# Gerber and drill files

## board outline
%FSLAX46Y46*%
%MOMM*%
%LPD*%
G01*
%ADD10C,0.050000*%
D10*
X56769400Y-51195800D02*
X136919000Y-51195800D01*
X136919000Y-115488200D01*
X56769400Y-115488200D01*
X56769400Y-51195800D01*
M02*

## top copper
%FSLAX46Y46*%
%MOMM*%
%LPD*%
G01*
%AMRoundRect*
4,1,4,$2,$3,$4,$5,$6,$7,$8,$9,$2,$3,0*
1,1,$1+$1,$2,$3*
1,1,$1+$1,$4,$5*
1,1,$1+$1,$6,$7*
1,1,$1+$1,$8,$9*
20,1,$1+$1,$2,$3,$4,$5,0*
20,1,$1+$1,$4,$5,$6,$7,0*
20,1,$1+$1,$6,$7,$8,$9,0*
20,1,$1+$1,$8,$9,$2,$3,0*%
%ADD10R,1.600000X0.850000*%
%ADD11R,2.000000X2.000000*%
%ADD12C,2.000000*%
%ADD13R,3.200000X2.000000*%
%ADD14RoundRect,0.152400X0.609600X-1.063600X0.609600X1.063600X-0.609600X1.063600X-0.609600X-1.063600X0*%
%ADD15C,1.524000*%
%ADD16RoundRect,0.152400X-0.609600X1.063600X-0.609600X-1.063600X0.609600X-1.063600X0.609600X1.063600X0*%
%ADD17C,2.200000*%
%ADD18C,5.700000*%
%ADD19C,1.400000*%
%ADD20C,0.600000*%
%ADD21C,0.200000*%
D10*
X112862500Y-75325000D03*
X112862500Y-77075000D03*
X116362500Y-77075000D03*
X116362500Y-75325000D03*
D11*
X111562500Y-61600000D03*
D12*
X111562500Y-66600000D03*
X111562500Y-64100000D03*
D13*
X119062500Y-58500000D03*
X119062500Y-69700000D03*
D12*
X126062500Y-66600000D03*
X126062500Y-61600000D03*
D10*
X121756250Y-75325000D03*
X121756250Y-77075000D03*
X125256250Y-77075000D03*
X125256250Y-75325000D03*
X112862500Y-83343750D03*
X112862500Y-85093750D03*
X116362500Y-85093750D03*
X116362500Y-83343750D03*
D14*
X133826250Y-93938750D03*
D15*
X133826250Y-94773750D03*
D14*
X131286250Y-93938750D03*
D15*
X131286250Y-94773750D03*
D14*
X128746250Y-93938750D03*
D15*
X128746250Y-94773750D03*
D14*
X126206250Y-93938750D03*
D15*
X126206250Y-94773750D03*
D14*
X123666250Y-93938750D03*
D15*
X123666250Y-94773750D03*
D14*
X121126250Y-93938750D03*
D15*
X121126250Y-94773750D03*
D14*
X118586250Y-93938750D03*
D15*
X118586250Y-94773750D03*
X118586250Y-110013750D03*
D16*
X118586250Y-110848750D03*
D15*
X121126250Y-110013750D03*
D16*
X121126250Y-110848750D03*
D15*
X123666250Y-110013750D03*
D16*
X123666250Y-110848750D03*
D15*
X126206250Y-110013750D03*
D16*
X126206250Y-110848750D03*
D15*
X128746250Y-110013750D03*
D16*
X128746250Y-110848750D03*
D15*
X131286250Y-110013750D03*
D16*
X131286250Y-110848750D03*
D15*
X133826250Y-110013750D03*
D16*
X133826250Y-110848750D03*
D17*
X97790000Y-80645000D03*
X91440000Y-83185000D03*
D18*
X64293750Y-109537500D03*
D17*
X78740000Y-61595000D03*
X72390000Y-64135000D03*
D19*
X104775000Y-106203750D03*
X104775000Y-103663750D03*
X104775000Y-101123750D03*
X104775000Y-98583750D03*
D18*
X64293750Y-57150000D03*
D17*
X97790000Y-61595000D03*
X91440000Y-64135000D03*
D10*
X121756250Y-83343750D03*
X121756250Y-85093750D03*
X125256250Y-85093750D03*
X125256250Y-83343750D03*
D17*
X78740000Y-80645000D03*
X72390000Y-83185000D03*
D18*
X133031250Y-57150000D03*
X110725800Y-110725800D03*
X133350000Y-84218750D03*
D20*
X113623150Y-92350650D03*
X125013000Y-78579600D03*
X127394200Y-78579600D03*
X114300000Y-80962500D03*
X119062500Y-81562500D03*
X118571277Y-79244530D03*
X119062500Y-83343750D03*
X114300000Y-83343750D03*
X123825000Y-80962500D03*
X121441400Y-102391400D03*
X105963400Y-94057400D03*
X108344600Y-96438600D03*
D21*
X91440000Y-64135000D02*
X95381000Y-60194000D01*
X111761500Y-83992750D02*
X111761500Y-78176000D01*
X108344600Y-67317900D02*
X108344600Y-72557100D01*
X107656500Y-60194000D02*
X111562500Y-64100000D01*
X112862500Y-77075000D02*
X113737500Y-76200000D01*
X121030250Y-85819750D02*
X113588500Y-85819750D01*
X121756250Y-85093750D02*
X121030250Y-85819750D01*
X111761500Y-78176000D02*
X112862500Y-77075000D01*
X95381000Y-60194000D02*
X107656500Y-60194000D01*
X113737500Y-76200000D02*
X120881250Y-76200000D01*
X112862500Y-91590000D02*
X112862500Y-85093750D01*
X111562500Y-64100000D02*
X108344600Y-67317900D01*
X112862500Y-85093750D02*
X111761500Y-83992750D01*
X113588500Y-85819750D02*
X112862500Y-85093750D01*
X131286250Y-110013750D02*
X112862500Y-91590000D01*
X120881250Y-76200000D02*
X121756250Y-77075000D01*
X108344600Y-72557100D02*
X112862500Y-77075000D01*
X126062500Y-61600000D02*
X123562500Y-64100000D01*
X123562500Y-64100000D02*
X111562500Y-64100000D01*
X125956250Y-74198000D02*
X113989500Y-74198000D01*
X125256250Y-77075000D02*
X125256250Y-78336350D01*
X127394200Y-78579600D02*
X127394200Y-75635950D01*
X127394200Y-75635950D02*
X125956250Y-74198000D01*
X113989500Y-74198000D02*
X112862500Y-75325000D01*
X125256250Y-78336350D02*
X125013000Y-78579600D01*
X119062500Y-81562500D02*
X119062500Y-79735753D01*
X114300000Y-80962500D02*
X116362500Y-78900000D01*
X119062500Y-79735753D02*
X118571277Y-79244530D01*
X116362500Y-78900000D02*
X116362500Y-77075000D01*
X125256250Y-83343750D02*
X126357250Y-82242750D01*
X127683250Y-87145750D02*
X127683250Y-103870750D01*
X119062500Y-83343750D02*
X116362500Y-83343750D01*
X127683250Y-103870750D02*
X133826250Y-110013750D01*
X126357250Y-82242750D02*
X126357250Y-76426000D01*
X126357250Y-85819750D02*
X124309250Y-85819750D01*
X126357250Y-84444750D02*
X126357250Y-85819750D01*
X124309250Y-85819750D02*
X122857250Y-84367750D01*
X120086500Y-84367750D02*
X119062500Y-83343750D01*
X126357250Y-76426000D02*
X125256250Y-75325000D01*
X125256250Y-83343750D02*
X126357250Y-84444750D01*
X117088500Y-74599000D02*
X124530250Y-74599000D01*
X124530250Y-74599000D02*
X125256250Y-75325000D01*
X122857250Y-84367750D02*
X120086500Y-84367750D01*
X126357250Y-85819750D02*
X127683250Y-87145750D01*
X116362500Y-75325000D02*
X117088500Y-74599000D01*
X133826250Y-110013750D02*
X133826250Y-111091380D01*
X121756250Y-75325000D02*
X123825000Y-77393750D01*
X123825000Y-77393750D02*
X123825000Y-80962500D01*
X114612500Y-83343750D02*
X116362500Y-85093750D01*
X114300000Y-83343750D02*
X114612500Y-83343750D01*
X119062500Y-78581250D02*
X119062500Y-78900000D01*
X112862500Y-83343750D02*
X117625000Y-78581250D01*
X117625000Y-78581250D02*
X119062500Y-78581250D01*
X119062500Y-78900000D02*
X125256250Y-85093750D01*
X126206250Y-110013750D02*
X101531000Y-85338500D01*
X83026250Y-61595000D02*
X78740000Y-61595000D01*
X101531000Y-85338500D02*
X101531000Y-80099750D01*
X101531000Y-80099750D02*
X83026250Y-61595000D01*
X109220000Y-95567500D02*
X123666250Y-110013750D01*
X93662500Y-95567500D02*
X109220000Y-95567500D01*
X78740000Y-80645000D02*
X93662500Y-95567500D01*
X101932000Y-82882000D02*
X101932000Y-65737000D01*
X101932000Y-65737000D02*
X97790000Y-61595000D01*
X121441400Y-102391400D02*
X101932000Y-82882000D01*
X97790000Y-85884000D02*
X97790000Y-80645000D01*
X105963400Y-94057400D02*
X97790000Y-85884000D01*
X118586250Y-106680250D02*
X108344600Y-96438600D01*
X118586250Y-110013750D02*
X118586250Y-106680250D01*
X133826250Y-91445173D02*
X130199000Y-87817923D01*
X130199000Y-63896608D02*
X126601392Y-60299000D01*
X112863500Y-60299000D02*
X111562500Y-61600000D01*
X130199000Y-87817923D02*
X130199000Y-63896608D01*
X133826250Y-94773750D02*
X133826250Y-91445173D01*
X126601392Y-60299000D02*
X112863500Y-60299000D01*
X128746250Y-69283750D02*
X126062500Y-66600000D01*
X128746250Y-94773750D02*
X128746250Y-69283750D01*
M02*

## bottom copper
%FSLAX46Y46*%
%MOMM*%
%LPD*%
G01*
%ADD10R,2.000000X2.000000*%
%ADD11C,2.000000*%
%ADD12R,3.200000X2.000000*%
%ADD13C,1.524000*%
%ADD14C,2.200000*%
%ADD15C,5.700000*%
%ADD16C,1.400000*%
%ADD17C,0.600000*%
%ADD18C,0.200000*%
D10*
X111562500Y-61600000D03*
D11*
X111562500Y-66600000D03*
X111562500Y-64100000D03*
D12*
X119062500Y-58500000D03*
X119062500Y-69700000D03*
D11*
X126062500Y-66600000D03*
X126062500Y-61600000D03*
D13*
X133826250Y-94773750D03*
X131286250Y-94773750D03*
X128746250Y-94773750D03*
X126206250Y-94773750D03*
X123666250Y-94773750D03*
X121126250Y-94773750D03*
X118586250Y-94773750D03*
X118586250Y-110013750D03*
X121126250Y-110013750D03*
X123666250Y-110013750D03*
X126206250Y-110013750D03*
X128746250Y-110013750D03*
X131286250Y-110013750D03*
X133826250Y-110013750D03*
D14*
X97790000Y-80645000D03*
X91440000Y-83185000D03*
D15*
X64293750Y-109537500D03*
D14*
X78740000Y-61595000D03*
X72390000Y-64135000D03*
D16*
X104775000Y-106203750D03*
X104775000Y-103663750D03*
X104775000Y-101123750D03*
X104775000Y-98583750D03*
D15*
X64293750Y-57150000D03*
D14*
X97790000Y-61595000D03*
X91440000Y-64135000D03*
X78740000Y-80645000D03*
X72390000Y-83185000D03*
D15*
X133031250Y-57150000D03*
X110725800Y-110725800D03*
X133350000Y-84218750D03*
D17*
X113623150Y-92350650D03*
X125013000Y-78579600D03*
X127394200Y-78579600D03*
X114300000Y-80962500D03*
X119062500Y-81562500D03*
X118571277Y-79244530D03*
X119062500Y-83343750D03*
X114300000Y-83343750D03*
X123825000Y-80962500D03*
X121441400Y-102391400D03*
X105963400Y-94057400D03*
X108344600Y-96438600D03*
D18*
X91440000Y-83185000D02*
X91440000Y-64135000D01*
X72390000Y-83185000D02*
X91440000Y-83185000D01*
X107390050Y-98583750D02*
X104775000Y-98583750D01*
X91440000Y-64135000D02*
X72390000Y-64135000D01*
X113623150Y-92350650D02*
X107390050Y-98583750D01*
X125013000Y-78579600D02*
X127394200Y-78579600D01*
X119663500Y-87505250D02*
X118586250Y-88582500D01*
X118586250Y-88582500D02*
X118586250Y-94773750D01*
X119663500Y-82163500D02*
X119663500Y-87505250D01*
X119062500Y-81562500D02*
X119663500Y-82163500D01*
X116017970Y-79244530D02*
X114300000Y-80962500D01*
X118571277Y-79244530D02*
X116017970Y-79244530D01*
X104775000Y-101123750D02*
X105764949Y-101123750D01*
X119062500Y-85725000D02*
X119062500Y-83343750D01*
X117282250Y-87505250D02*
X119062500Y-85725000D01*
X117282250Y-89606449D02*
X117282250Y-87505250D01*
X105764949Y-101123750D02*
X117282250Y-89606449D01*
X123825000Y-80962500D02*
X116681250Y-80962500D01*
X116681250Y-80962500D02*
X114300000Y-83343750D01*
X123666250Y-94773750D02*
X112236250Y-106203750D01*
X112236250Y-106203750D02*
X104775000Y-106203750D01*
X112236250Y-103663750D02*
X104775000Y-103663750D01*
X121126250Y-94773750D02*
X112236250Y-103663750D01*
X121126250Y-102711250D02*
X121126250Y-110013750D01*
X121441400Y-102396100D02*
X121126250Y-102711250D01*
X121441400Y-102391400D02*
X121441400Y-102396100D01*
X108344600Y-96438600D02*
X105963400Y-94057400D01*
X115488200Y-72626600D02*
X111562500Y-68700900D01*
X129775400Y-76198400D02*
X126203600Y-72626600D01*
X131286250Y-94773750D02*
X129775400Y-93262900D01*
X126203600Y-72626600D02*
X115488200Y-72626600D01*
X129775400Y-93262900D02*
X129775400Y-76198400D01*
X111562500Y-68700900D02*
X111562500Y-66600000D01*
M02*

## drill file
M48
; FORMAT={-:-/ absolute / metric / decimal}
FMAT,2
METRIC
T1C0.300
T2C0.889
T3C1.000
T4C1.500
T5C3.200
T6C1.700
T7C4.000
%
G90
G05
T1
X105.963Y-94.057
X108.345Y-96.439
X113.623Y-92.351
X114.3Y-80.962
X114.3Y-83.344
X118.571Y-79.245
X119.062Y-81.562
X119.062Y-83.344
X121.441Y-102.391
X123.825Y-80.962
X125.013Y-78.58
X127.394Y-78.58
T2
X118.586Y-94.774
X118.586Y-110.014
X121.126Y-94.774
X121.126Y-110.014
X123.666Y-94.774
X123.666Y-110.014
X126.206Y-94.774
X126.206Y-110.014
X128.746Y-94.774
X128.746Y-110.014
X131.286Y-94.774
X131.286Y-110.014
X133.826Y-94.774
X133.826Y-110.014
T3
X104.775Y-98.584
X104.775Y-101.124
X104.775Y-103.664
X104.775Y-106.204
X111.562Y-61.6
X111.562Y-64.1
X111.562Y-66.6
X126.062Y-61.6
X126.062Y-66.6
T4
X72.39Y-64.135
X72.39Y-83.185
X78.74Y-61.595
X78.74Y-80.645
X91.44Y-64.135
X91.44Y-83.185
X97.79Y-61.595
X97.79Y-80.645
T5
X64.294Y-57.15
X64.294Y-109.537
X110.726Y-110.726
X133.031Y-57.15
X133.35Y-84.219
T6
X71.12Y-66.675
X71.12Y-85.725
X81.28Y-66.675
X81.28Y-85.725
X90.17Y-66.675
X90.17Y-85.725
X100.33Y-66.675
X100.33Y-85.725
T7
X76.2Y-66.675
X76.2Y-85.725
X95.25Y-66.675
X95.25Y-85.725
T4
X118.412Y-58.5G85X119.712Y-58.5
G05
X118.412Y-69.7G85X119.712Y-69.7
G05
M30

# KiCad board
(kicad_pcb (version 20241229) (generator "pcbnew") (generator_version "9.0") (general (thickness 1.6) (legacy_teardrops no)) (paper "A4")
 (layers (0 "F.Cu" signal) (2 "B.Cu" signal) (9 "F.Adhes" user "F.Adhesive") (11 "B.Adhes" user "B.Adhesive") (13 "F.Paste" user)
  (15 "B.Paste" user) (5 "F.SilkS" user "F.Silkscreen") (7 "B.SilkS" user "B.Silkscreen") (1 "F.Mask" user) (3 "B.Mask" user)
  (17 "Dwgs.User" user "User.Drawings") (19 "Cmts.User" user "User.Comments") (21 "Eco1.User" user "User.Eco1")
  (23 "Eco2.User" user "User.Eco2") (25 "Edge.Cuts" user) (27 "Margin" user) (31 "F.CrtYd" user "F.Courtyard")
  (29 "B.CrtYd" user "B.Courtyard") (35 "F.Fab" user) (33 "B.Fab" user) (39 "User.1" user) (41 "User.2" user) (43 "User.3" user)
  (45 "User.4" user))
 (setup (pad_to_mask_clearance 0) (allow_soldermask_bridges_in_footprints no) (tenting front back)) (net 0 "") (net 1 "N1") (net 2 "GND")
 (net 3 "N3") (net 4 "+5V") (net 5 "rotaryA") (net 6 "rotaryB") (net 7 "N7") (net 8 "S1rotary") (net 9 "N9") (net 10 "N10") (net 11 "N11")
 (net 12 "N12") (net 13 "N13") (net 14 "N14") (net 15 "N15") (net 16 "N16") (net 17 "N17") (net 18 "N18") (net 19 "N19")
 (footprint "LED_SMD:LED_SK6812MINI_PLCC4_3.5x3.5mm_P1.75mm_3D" (layer "F.Cu") (at 114.6125 76.2)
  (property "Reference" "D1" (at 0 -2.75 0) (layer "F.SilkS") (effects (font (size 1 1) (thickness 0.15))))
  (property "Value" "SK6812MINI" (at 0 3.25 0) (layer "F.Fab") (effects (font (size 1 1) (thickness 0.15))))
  (pad "1" smd rect (at -1.75 -0.875) (size 1.6 0.85) (layers "F.Cu" "F.Mask" "F.Paste") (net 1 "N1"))
  (pad "2" smd rect (at -1.75 0.875) (size 1.6 0.85) (layers "F.Cu" "F.Mask" "F.Paste") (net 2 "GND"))
  (pad "3" smd rect (at 1.75 0.875) (size 1.6 0.85) (layers "F.Cu" "F.Mask" "F.Paste") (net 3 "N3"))
  (pad "4" smd rect (at 1.75 -0.875) (size 1.6 0.85) (layers "F.Cu" "F.Mask" "F.Paste") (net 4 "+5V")))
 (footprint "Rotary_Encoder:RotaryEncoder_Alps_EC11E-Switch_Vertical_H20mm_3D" (layer "F.Cu") (at 111.5625 61.6)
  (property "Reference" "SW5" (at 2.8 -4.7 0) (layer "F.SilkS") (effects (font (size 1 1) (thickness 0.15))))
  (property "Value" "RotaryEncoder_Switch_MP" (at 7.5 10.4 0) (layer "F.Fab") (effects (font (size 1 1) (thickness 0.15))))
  (pad "A" thru_hole rect (at 0 0) (size 2 2) (drill 1) (layers "*.Cu" "*.Mask") (remove_unused_layers no) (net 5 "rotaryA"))
  (pad "B" thru_hole circle (at 0 5) (size 2 2) (drill 1) (layers "*.Cu" "*.Mask") (remove_unused_layers no) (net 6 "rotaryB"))
  (pad "C" thru_hole circle (at 0 2.5) (size 2 2) (drill 1) (layers "*.Cu" "*.Mask") (remove_unused_layers no) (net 2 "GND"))
  (pad "MP" thru_hole rect (at 7.5 -3.1) (size 3.2 2) (drill oval 2.8 1.5) (layers "*.Cu" "*.Mask") (remove_unused_layers no) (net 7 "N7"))
  (pad "MP" thru_hole rect (at 7.5 8.1) (size 3.2 2) (drill oval 2.8 1.5) (layers "*.Cu" "*.Mask") (remove_unused_layers no) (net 7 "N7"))
  (pad "S1" thru_hole circle (at 14.5 5) (size 2 2) (drill 1) (layers "*.Cu" "*.Mask") (remove_unused_layers no) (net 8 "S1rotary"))
  (pad "S2" thru_hole circle (at 14.5 0) (size 2 2) (drill 1) (layers "*.Cu" "*.Mask") (remove_unused_layers no) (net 2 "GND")))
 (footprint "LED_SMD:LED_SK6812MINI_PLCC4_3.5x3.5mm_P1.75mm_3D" (layer "F.Cu") (at 123.50625 76.2)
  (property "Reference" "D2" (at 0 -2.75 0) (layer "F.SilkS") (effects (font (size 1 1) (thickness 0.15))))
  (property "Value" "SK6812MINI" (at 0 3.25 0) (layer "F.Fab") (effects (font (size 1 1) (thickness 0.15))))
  (pad "1" smd rect (at -1.75 -0.875) (size 1.6 0.85) (layers "F.Cu" "F.Mask" "F.Paste") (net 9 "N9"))
  (pad "2" smd rect (at -1.75 0.875) (size 1.6 0.85) (layers "F.Cu" "F.Mask" "F.Paste") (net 2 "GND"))
  (pad "3" smd rect (at 1.75 0.875) (size 1.6 0.85) (layers "F.Cu" "F.Mask" "F.Paste") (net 1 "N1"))
  (pad "4" smd rect (at 1.75 -0.875) (size 1.6 0.85) (layers "F.Cu" "F.Mask" "F.Paste") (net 4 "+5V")))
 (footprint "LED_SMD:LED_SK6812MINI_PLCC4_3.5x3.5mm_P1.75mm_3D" (layer "F.Cu") (at 114.6125 84.21875)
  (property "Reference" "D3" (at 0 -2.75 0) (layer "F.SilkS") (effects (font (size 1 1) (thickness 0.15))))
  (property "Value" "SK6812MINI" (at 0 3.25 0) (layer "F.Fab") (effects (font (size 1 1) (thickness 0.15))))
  (pad "1" smd rect (at -1.75 -0.875) (size 1.6 0.85) (layers "F.Cu" "F.Mask" "F.Paste") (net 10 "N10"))
  (pad "2" smd rect (at -1.75 0.875) (size 1.6 0.85) (layers "F.Cu" "F.Mask" "F.Paste") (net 2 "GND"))
  (pad "3" smd rect (at 1.75 0.875) (size 1.6 0.85) (layers "F.Cu" "F.Mask" "F.Paste") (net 9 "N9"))
  (pad "4" smd rect (at 1.75 -0.875) (size 1.6 0.85) (layers "F.Cu" "F.Mask" "F.Paste") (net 4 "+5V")))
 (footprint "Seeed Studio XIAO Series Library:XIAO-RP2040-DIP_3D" (layer "F.Cu") (at 126.20625 102.39375 -90)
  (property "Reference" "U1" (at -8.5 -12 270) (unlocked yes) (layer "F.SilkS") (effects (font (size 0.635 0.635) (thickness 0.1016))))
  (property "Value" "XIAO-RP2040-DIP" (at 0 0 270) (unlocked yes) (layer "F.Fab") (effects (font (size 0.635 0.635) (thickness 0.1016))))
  (pad "1" smd roundrect (at -8.455 -7.62 90) (size 2.432 1.524) (layers "F.Cu" "F.Mask") (roundrect_rratio 0.1) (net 5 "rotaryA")
   (thermal_bridge_angle 45))
  (pad "1" thru_hole circle (at -7.62 -7.62 90) (size 1.524 1.524) (drill 0.889) (layers "*.Cu" "*.Mask") (remove_unused_layers no)
   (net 5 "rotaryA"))
  (pad "2" smd roundrect (at -8.455 -5.08 90) (size 2.432 1.524) (layers "F.Cu" "F.Mask") (roundrect_rratio 0.1) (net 6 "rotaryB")
   (thermal_bridge_angle 45))
  (pad "2" thru_hole circle (at -7.62 -5.08 90) (size 1.524 1.524) (drill 0.889) (layers "*.Cu" "*.Mask") (remove_unused_layers no)
   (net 6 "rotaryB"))
  (pad "3" smd roundrect (at -8.455 -2.54 90) (size 2.432 1.524) (layers "F.Cu" "F.Mask") (roundrect_rratio 0.1) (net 8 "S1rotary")
   (thermal_bridge_angle 45))
  (pad "3" thru_hole circle (at -7.62 -2.54 90) (size 1.524 1.524) (drill 0.889) (layers "*.Cu" "*.Mask") (remove_unused_layers no)
   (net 8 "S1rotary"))
  (pad "4" smd roundrect (at -8.455 0 90) (size 2.432 1.524) (layers "F.Cu" "F.Mask") (roundrect_rratio 0.1) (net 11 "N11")
   (thermal_bridge_angle 45))
  (pad "4" thru_hole circle (at -7.62 0 90) (size 1.524 1.524) (drill 0.889) (layers "*.Cu" "*.Mask") (remove_unused_layers no)
   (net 11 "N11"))
  (pad "5" smd roundrect (at -8.455 2.54 90) (size 2.432 1.524) (layers "F.Cu" "F.Mask") (roundrect_rratio 0.1) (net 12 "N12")
   (thermal_bridge_angle 45))
  (pad "5" thru_hole circle (at -7.62 2.54 90) (size 1.524 1.524) (drill 0.889) (layers "*.Cu" "*.Mask") (remove_unused_layers no)
   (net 12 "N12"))
  (pad "6" smd roundrect (at -8.455 5.08 90) (size 2.432 1.524) (layers "F.Cu" "F.Mask") (roundrect_rratio 0.1) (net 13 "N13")
   (thermal_bridge_angle 45))
  (pad "6" thru_hole circle (at -7.62 5.08 90) (size 1.524 1.524) (drill 0.889) (layers "*.Cu" "*.Mask") (remove_unused_layers no)
   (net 13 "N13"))
  (pad "7" smd roundrect (at -8.455 7.62 90) (size 2.432 1.524) (layers "F.Cu" "F.Mask") (roundrect_rratio 0.1) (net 3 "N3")
   (thermal_bridge_angle 45))
  (pad "7" thru_hole circle (at -7.62 7.62 90) (size 1.524 1.524) (drill 0.889) (layers "*.Cu" "*.Mask") (remove_unused_layers no)
   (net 3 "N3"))
  (pad "8" thru_hole circle (at 7.62 7.62 270) (size 1.524 1.524) (drill 0.889) (layers "*.Cu" "*.Mask") (remove_unused_layers no)
   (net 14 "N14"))
  (pad "8" smd roundrect (at 8.455 7.62 270) (size 2.432 1.524) (layers "F.Cu" "F.Mask") (roundrect_rratio 0.1) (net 14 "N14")
   (thermal_bridge_angle 45))
  (pad "9" thru_hole circle (at 7.62 5.08 270) (size 1.524 1.524) (drill 0.889) (layers "*.Cu" "*.Mask") (remove_unused_layers no)
   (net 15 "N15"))
  (pad "9" smd roundrect (at 8.455 5.08 270) (size 2.432 1.524) (layers "F.Cu" "F.Mask") (roundrect_rratio 0.1) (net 15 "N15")
   (thermal_bridge_angle 45))
  (pad "10" thru_hole circle (at 7.62 2.54 270) (size 1.524 1.524) (drill 0.889) (layers "*.Cu" "*.Mask") (remove_unused_layers no)
   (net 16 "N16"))
  (pad "10" smd roundrect (at 8.455 2.54 270) (size 2.432 1.524) (layers "F.Cu" "F.Mask") (roundrect_rratio 0.1) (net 16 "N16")
   (thermal_bridge_angle 45))
  (pad "11" thru_hole circle (at 7.62 0 270) (size 1.524 1.524) (drill 0.889) (layers "*.Cu" "*.Mask") (remove_unused_layers no)
   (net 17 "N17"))
  (pad "11" smd roundrect (at 8.455 0 270) (size 2.432 1.524) (layers "F.Cu" "F.Mask") (roundrect_rratio 0.1) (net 17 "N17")
   (thermal_bridge_angle 45))
  (pad "12" thru_hole circle (at 7.62 -2.54 270) (size 1.524 1.524) (drill 0.889) (layers "*.Cu" "*.Mask") (remove_unused_layers no)
   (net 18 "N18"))
  (pad "12" smd roundrect (at 8.455 -2.54 270) (size 2.432 1.524) (layers "F.Cu" "F.Mask") (roundrect_rratio 0.1) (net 18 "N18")
   (thermal_bridge_angle 45))
  (pad "13" thru_hole circle (at 7.62 -5.08 270) (size 1.524 1.524) (drill 0.889) (layers "*.Cu" "*.Mask") (remove_unused_layers no)
   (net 2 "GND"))
  (pad "13" smd roundrect (at 8.455 -5.08 270) (size 2.432 1.524) (layers "F.Cu" "F.Mask") (roundrect_rratio 0.1) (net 2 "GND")
   (thermal_bridge_angle 45))
  (pad "14" thru_hole circle (at 7.62 -7.62 270) (size 1.524 1.524) (drill 0.889) (layers "*.Cu" "*.Mask") (remove_unused_layers no)
   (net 4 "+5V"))
  (pad "14" smd roundrect (at 8.455 -7.62 270) (size 2.432 1.524) (layers "F.Cu" "F.Mask") (roundrect_rratio 0.1) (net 4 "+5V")
   (thermal_bridge_angle 45)))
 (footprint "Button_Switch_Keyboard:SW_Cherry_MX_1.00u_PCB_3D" (layer "F.Cu") (at 97.79 80.645)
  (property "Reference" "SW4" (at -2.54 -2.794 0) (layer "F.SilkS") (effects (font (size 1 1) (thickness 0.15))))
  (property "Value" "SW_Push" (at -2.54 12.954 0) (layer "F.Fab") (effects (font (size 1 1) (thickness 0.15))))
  (pad "" np_thru_hole circle (at -7.62 5.08) (size 1.7 1.7) (drill 1.7) (layers "*.Cu" "*.Mask"))
  (pad "" np_thru_hole circle (at -2.54 5.08) (size 4 4) (drill 4) (layers "*.Cu" "*.Mask"))
  (pad "" np_thru_hole circle (at 2.54 5.08) (size 1.7 1.7) (drill 1.7) (layers "*.Cu" "*.Mask"))
  (pad "1" thru_hole circle (at 0 0) (size 2.2 2.2) (drill 1.5) (layers "*.Cu" "*.Mask") (remove_unused_layers no) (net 14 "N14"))
  (pad "2" thru_hole circle (at -6.35 2.54) (size 2.2 2.2) (drill 1.5) (layers "*.Cu" "*.Mask") (remove_unused_layers no) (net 2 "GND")))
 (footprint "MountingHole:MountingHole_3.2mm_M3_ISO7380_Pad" (layer "F.Cu") (at 64.29375 109.5375)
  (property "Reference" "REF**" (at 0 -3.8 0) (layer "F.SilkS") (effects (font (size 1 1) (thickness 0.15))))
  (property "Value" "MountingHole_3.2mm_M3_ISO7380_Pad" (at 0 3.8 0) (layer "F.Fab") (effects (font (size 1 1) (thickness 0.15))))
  (pad "1" thru_hole circle (at 0 0) (size 5.7 5.7) (drill 3.2) (layers "*.Cu" "*.Mask") (remove_unused_layers no) (zone_connect 2)))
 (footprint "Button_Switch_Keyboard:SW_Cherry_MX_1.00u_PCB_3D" (layer "F.Cu") (at 78.74 61.595)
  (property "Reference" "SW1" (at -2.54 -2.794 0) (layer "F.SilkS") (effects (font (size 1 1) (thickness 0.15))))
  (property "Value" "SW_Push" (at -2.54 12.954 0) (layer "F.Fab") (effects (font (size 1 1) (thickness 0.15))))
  (pad "" np_thru_hole circle (at -7.62 5.08) (size 1.7 1.7) (drill 1.7) (layers "*.Cu" "*.Mask"))
  (pad "" np_thru_hole circle (at -2.54 5.08) (size 4 4) (drill 4) (layers "*.Cu" "*.Mask"))
  (pad "" np_thru_hole circle (at 2.54 5.08) (size 1.7 1.7) (drill 1.7) (layers "*.Cu" "*.Mask"))
  (pad "1" thru_hole circle (at 0 0) (size 2.2 2.2) (drill 1.5) (layers "*.Cu" "*.Mask") (remove_unused_layers no) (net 17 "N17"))
  (pad "2" thru_hole circle (at -6.35 2.54) (size 2.2 2.2) (drill 1.5) (layers "*.Cu" "*.Mask") (remove_unused_layers no) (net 2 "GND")))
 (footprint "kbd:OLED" (layer "F.Cu") (at 104.775 102.39375 90)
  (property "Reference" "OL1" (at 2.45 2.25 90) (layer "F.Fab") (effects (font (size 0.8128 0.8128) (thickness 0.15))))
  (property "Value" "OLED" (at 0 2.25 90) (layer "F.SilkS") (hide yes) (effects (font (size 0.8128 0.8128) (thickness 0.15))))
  (pad "1" thru_hole circle (at -3.81 0 90) (size 1.4 1.4) (drill 1) (layers "*.Cu" "*.Mask") (remove_unused_layers no) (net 12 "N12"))
  (pad "2" thru_hole circle (at -1.27 0 90) (size 1.4 1.4) (drill 1) (layers "*.Cu" "*.Mask") (remove_unused_layers no) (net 13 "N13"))
  (pad "3" thru_hole circle (at 1.27 0 90) (size 1.4 1.4) (drill 1) (layers "*.Cu" "*.Mask") (remove_unused_layers no) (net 4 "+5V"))
  (pad "4" thru_hole circle (at 3.81 0 90) (size 1.4 1.4) (drill 1) (layers "*.Cu" "*.Mask") (remove_unused_layers no) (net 2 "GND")))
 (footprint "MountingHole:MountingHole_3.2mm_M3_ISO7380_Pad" (layer "F.Cu") (at 64.29375 57.15)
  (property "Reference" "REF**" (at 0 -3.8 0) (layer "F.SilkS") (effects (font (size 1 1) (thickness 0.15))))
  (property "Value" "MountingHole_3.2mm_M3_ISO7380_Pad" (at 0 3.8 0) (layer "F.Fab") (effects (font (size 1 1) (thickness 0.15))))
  (pad "1" thru_hole circle (at 0 0) (size 5.7 5.7) (drill 3.2) (layers "*.Cu" "*.Mask") (remove_unused_layers no) (zone_connect 2)))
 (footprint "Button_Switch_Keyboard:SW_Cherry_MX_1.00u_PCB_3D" (layer "F.Cu") (at 97.79 61.595)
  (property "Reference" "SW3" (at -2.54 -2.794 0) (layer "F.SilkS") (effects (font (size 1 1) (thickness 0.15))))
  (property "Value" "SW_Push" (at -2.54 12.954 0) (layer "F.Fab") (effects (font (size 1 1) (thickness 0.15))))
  (pad "" np_thru_hole circle (at -7.62 5.08) (size 1.7 1.7) (drill 1.7) (layers "*.Cu" "*.Mask"))
  (pad "" np_thru_hole circle (at -2.54 5.08) (size 4 4) (drill 4) (layers "*.Cu" "*.Mask"))
  (pad "" np_thru_hole circle (at 2.54 5.08) (size 1.7 1.7) (drill 1.7) (layers "*.Cu" "*.Mask"))
  (pad "1" thru_hole circle (at 0 0) (size 2.2 2.2) (drill 1.5) (layers "*.Cu" "*.Mask") (remove_unused_layers no) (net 15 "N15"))
  (pad "2" thru_hole circle (at -6.35 2.54) (size 2.2 2.2) (drill 1.5) (layers "*.Cu" "*.Mask") (remove_unused_layers no) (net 2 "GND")))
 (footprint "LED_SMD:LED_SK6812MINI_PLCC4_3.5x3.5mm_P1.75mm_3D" (layer "F.Cu") (at 123.50625 84.21875)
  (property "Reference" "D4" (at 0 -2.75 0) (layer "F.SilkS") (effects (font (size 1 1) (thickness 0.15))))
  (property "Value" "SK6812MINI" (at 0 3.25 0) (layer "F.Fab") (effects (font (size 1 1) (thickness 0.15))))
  (pad "1" smd rect (at -1.75 -0.875) (size 1.6 0.85) (layers "F.Cu" "F.Mask" "F.Paste") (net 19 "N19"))
  (pad "2" smd rect (at -1.75 0.875) (size 1.6 0.85) (layers "F.Cu" "F.Mask" "F.Paste") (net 2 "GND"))
  (pad "3" smd rect (at 1.75 0.875) (size 1.6 0.85) (layers "F.Cu" "F.Mask" "F.Paste") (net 10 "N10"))
  (pad "4" smd rect (at 1.75 -0.875) (size 1.6 0.85) (layers "F.Cu" "F.Mask" "F.Paste") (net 4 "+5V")))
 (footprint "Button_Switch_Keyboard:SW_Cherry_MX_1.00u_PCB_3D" (layer "F.Cu") (at 78.74 80.645)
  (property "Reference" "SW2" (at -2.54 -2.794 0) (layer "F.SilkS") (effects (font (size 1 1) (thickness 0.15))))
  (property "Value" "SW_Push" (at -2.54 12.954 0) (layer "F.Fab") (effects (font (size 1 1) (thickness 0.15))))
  (pad "" np_thru_hole circle (at -7.62 5.08) (size 1.7 1.7) (drill 1.7) (layers "*.Cu" "*.Mask"))
  (pad "" np_thru_hole circle (at -2.54 5.08) (size 4 4) (drill 4) (layers "*.Cu" "*.Mask"))
  (pad "" np_thru_hole circle (at 2.54 5.08) (size 1.7 1.7) (drill 1.7) (layers "*.Cu" "*.Mask"))
  (pad "1" thru_hole circle (at 0 0) (size 2.2 2.2) (drill 1.5) (layers "*.Cu" "*.Mask") (remove_unused_layers no) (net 16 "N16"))
  (pad "2" thru_hole circle (at -6.35 2.54) (size 2.2 2.2) (drill 1.5) (layers "*.Cu" "*.Mask") (remove_unused_layers no) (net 2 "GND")))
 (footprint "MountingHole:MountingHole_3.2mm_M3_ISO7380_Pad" (layer "F.Cu") (at 133.03125 57.15)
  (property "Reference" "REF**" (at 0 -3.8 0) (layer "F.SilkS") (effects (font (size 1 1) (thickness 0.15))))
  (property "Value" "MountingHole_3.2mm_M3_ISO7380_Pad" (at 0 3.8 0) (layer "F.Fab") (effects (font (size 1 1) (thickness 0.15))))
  (pad "1" thru_hole circle (at 0 0) (size 5.7 5.7) (drill 3.2) (layers "*.Cu" "*.Mask") (remove_unused_layers no) (zone_connect 2)))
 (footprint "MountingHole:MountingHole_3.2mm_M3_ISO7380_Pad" (layer "F.Cu") (at 110.7258 110.7258)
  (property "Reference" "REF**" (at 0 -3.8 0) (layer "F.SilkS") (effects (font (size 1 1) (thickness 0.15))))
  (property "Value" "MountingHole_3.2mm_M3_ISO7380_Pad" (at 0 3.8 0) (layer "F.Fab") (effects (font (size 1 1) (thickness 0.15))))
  (pad "1" thru_hole circle (at 0 0) (size 5.7 5.7) (drill 3.2) (layers "*.Cu" "*.Mask") (remove_unused_layers no) (zone_connect 2)))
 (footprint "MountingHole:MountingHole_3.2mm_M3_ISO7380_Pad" (layer "F.Cu") (at 133.35 84.21875)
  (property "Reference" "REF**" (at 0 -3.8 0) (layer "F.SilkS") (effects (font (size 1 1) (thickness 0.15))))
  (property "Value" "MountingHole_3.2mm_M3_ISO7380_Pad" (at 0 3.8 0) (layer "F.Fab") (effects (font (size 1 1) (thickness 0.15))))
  (pad "1" thru_hole circle (at 0 0) (size 5.7 5.7) (drill 3.2) (layers "*.Cu" "*.Mask") (remove_unused_layers no) (zone_connect 2)))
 (gr_rect (start 56.7694 51.1958) (end 136.919 115.4882) (stroke (width 0.05) (type default)) (fill no) (layer "Edge.Cuts"))
 (segment (start 91.44 64.135) (end 95.381 60.194) (width 0.2) (layer "F.Cu") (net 2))
 (segment (start 111.7615 83.99275) (end 111.7615 78.176) (width 0.2) (layer "F.Cu") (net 2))
 (segment (start 108.3446 67.3179) (end 108.3446 72.5571) (width 0.2) (layer "F.Cu") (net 2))
 (segment (start 107.6565 60.194) (end 111.5625 64.1) (width 0.2) (layer "F.Cu") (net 2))
 (segment (start 112.8625 77.075) (end 113.7375 76.2) (width 0.2) (layer "F.Cu") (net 2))
 (segment (start 121.03025 85.81975) (end 113.5885 85.81975) (width 0.2) (layer "F.Cu") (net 2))
 (segment (start 121.75625 85.09375) (end 121.03025 85.81975) (width 0.2) (layer "F.Cu") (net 2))
 (segment (start 111.7615 78.176) (end 112.8625 77.075) (width 0.2) (layer "F.Cu") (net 2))
 (segment (start 95.381 60.194) (end 107.6565 60.194) (width 0.2) (layer "F.Cu") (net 2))
 (segment (start 113.7375 76.2) (end 120.88125 76.2) (width 0.2) (layer "F.Cu") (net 2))
 (segment (start 112.8625 91.59) (end 112.8625 85.09375) (width 0.2) (layer "F.Cu") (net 2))
 (segment (start 111.5625 64.1) (end 108.3446 67.3179) (width 0.2) (layer "F.Cu") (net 2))
 (segment (start 112.8625 85.09375) (end 111.7615 83.99275) (width 0.2) (layer "F.Cu") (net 2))
 (segment (start 113.5885 85.81975) (end 112.8625 85.09375) (width 0.2) (layer "F.Cu") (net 2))
 (segment (start 131.28625 110.01375) (end 112.8625 91.59) (width 0.2) (layer "F.Cu") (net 2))
 (segment (start 120.88125 76.2) (end 121.75625 77.075) (width 0.2) (layer "F.Cu") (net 2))
 (segment (start 108.3446 72.5571) (end 112.8625 77.075) (width 0.2) (layer "F.Cu") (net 2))
 (segment (start 126.0625 61.6) (end 123.5625 64.1) (width 0.2) (layer "F.Cu") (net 2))
 (segment (start 123.5625 64.1) (end 111.5625 64.1) (width 0.2) (layer "F.Cu") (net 2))
 (via (at 113.62315 92.35065) (size 0.6) (drill 0.3) (layers "F.Cu" "B.Cu") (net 2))
 (segment (start 91.44 83.185) (end 91.44 64.135) (width 0.2) (layer "B.Cu") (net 2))
 (segment (start 72.39 83.185) (end 91.44 83.185) (width 0.2) (layer "B.Cu") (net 2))
 (segment (start 107.39005 98.58375) (end 104.775 98.58375) (width 0.2) (layer "B.Cu") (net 2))
 (segment (start 91.44 64.135) (end 72.39 64.135) (width 0.2) (layer "B.Cu") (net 2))
 (segment (start 113.62315 92.35065) (end 107.39005 98.58375) (width 0.2) (layer "B.Cu") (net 2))
 (segment (start 125.95625 74.198) (end 113.9895 74.198) (width 0.2) (layer "F.Cu") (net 1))
 (segment (start 125.25625 77.075) (end 125.25625 78.33635) (width 0.2) (layer "F.Cu") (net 1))
 (segment (start 127.3942 78.5796) (end 127.3942 75.63595) (width 0.2) (layer "F.Cu") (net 1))
 (segment (start 127.3942 75.63595) (end 125.95625 74.198) (width 0.2) (layer "F.Cu") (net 1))
 (segment (start 113.9895 74.198) (end 112.8625 75.325) (width 0.2) (layer "F.Cu") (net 1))
 (segment (start 125.25625 78.33635) (end 125.013 78.5796) (width 0.2) (layer "F.Cu") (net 1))
 (via (at 125.013 78.5796) (size 0.6) (drill 0.3) (layers "F.Cu" "B.Cu") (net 1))
 (via (at 127.3942 78.5796) (size 0.6) (drill 0.3) (layers "F.Cu" "B.Cu") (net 1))
 (segment (start 125.013 78.5796) (end 127.3942 78.5796) (width 0.2) (layer "B.Cu") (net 1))
 (segment (start 119.0625 81.5625) (end 119.0625 79.735753) (width 0.2) (layer "F.Cu") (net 3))
 (segment (start 114.3 80.9625) (end 116.3625 78.9) (width 0.2) (layer "F.Cu") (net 3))
 (segment (start 119.0625 79.735753) (end 118.571277 79.24453) (width 0.2) (layer "F.Cu") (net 3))
 (segment (start 116.3625 78.9) (end 116.3625 77.075) (width 0.2) (layer "F.Cu") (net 3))
 (via (at 114.3 80.9625) (size 0.6) (drill 0.3) (layers "F.Cu" "B.Cu") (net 3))
 (via (at 119.0625 81.5625) (size 0.6) (drill 0.3) (layers "F.Cu" "B.Cu") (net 3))
 (via (at 118.571277 79.24453) (size 0.6) (drill 0.3) (layers "F.Cu" "B.Cu") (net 3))
 (segment (start 119.6635 87.50525) (end 118.58625 88.5825) (width 0.2) (layer "B.Cu") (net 3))
 (segment (start 118.58625 88.5825) (end 118.58625 94.77375) (width 0.2) (layer "B.Cu") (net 3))
 (segment (start 119.6635 82.1635) (end 119.6635 87.50525) (width 0.2) (layer "B.Cu") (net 3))
 (segment (start 119.0625 81.5625) (end 119.6635 82.1635) (width 0.2) (layer "B.Cu") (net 3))
 (segment (start 116.01797 79.24453) (end 114.3 80.9625) (width 0.2) (layer "B.Cu") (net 3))
 (segment (start 118.571277 79.24453) (end 116.01797 79.24453) (width 0.2) (layer "B.Cu") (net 3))
 (segment (start 125.25625 83.34375) (end 126.35725 82.24275) (width 0.2) (layer "F.Cu") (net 4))
 (segment (start 127.68325 87.14575) (end 127.68325 103.87075) (width 0.2) (layer "F.Cu") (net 4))
 (segment (start 119.0625 83.34375) (end 116.3625 83.34375) (width 0.2) (layer "F.Cu") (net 4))
 (segment (start 127.68325 103.87075) (end 133.82625 110.01375) (width 0.2) (layer "F.Cu") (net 4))
 (segment (start 126.35725 82.24275) (end 126.35725 76.426) (width 0.2) (layer "F.Cu") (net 4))
 (segment (start 126.35725 85.81975) (end 124.30925 85.81975) (width 0.2) (layer "F.Cu") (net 4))
 (segment (start 126.35725 84.44475) (end 126.35725 85.81975) (width 0.2) (layer "F.Cu") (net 4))
 (segment (start 124.30925 85.81975) (end 122.85725 84.36775) (width 0.2) (layer "F.Cu") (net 4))
 (segment (start 120.0865 84.36775) (end 119.0625 83.34375) (width 0.2) (layer "F.Cu") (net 4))
 (segment (start 126.35725 76.426) (end 125.25625 75.325) (width 0.2) (layer "F.Cu") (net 4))
 (segment (start 125.25625 83.34375) (end 126.35725 84.44475) (width 0.2) (layer "F.Cu") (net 4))
 (segment (start 117.0885 74.599) (end 124.53025 74.599) (width 0.2) (layer "F.Cu") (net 4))
 (segment (start 124.53025 74.599) (end 125.25625 75.325) (width 0.2) (layer "F.Cu") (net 4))
 (segment (start 122.85725 84.36775) (end 120.0865 84.36775) (width 0.2) (layer "F.Cu") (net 4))
 (segment (start 126.35725 85.81975) (end 127.68325 87.14575) (width 0.2) (layer "F.Cu") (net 4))
 (segment (start 116.3625 75.325) (end 117.0885 74.599) (width 0.2) (layer "F.Cu") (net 4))
 (segment (start 133.82625 110.01375) (end 133.82625 111.09138) (width 0.2) (layer "F.Cu") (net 4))
 (via (at 119.0625 83.34375) (size 0.6) (drill 0.3) (layers "F.Cu" "B.Cu") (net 4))
 (segment (start 104.775 101.12375) (end 105.764949 101.12375) (width 0.2) (layer "B.Cu") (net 4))
 (segment (start 119.0625 85.725) (end 119.0625 83.34375) (width 0.2) (layer "B.Cu") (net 4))
 (segment (start 117.28225 87.50525) (end 119.0625 85.725) (width 0.2) (layer "B.Cu") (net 4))
 (segment (start 117.28225 89.606449) (end 117.28225 87.50525) (width 0.2) (layer "B.Cu") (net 4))
 (segment (start 105.764949 101.12375) (end 117.28225 89.606449) (width 0.2) (layer "B.Cu") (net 4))
 (segment (start 121.75625 75.325) (end 123.825 77.39375) (width 0.2) (layer "F.Cu") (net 9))
 (segment (start 123.825 77.39375) (end 123.825 80.9625) (width 0.2) (layer "F.Cu") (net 9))
 (segment (start 114.6125 83.34375) (end 116.3625 85.09375) (width 0.2) (layer "F.Cu") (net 9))
 (segment (start 114.3 83.34375) (end 114.6125 83.34375) (width 0.2) (layer "F.Cu") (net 9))
 (via (at 114.3 83.34375) (size 0.6) (drill 0.3) (layers "F.Cu" "B.Cu") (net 9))
 (via (at 123.825 80.9625) (size 0.6) (drill 0.3) (layers "F.Cu" "B.Cu") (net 9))
 (segment (start 123.825 80.9625) (end 116.68125 80.9625) (width 0.2) (layer "B.Cu") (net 9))
 (segment (start 116.68125 80.9625) (end 114.3 83.34375) (width 0.2) (layer "B.Cu") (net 9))
 (segment (start 119.0625 78.58125) (end 119.0625 78.9) (width 0.2) (layer "F.Cu") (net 10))
 (segment (start 112.8625 83.34375) (end 117.625 78.58125) (width 0.2) (layer "F.Cu") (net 10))
 (segment (start 117.625 78.58125) (end 119.0625 78.58125) (width 0.2) (layer "F.Cu") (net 10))
 (segment (start 119.0625 78.9) (end 125.25625 85.09375) (width 0.2) (layer "F.Cu") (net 10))
 (segment (start 123.66625 94.77375) (end 112.23625 106.20375) (width 0.2) (layer "B.Cu") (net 12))
 (segment (start 112.23625 106.20375) (end 104.775 106.20375) (width 0.2) (layer "B.Cu") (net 12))
 (segment (start 112.23625 103.66375) (end 104.775 103.66375) (width 0.2) (layer "B.Cu") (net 13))
 (segment (start 121.12625 94.77375) (end 112.23625 103.66375) (width 0.2) (layer "B.Cu") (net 13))
 (segment (start 126.20625 110.01375) (end 101.531 85.3385) (width 0.2) (layer "F.Cu") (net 17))
 (segment (start 83.02625 61.595) (end 78.74 61.595) (width 0.2) (layer "F.Cu") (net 17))
 (segment (start 101.531 85.3385) (end 101.531 80.09975) (width 0.2) (layer "F.Cu") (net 17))
 (segment (start 101.531 80.09975) (end 83.02625 61.595) (width 0.2) (layer "F.Cu") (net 17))
 (segment (start 109.22 95.5675) (end 123.66625 110.01375) (width 0.2) (layer "F.Cu") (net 16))
 (segment (start 93.6625 95.5675) (end 109.22 95.5675) (width 0.2) (layer "F.Cu") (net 16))
 (segment (start 78.74 80.645) (end 93.6625 95.5675) (width 0.2) (layer "F.Cu") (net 16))
 (segment (start 101.932 82.882) (end 101.932 65.737) (width 0.2) (layer "F.Cu") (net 15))
 (segment (start 101.932 65.737) (end 97.79 61.595) (width 0.2) (layer "F.Cu") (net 15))
 (segment (start 121.4414 102.3914) (end 101.932 82.882) (width 0.2) (layer "F.Cu") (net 15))
 (via (at 121.4414 102.3914) (size 0.6) (drill 0.3) (layers "F.Cu" "B.Cu") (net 15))
 (segment (start 121.12625 102.71125) (end 121.12625 110.01375) (width 0.2) (layer "B.Cu") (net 15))
 (segment (start 121.4414 102.3961) (end 121.12625 102.71125) (width 0.2) (layer "B.Cu") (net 15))
 (segment (start 121.4414 102.3914) (end 121.4414 102.3961) (width 0.2) (layer "B.Cu") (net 15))
 (segment (start 97.79 85.884) (end 97.79 80.645) (width 0.2) (layer "F.Cu") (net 14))
 (segment (start 105.9634 94.0574) (end 97.79 85.884) (width 0.2) (layer "F.Cu") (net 14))
 (segment (start 118.58625 106.68025) (end 108.3446 96.4386) (width 0.2) (layer "F.Cu") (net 14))
 (segment (start 118.58625 110.01375) (end 118.58625 106.68025) (width 0.2) (layer "F.Cu") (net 14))
 (via (at 105.9634 94.0574) (size 0.6) (drill 0.3) (layers "F.Cu" "B.Cu") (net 14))
 (via (at 108.3446 96.4386) (size 0.6) (drill 0.3) (layers "F.Cu" "B.Cu") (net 14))
 (segment (start 108.3446 96.4386) (end 105.9634 94.0574) (width 0.2) (layer "B.Cu") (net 14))
 (segment (start 115.4882 72.6266) (end 111.5625 68.7009) (width 0.2) (layer "B.Cu") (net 6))
 (segment (start 129.7754 76.1984) (end 126.2036 72.6266) (width 0.2) (layer "B.Cu") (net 6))
 (segment (start 131.28625 94.77375) (end 129.7754 93.2629) (width 0.2) (layer "B.Cu") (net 6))
 (segment (start 126.2036 72.6266) (end 115.4882 72.6266) (width 0.2) (layer "B.Cu") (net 6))
 (segment (start 129.7754 93.2629) (end 129.7754 76.1984) (width 0.2) (layer "B.Cu") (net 6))
 (segment (start 111.5625 68.7009) (end 111.5625 66.6) (width 0.2) (layer "B.Cu") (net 6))
 (segment (start 133.82625 91.445173) (end 130.199 87.817923) (width 0.2) (layer "F.Cu") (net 5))
 (segment (start 130.199 63.896608) (end 126.601392 60.299) (width 0.2) (layer "F.Cu") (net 5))
 (segment (start 112.8635 60.299) (end 111.5625 61.6) (width 0.2) (layer "F.Cu") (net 5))
 (segment (start 130.199 87.817923) (end 130.199 63.896608) (width 0.2) (layer "F.Cu") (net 5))
 (segment (start 133.82625 94.77375) (end 133.82625 91.445173) (width 0.2) (layer "F.Cu") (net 5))
 (segment (start 126.601392 60.299) (end 112.8635 60.299) (width 0.2) (layer "F.Cu") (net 5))
 (segment (start 128.74625 69.28375) (end 126.0625 66.6) (width 0.2) (layer "F.Cu") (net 8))
 (segment (start 128.74625 94.77375) (end 128.74625 69.28375) (width 0.2) (layer "F.Cu") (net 8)))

